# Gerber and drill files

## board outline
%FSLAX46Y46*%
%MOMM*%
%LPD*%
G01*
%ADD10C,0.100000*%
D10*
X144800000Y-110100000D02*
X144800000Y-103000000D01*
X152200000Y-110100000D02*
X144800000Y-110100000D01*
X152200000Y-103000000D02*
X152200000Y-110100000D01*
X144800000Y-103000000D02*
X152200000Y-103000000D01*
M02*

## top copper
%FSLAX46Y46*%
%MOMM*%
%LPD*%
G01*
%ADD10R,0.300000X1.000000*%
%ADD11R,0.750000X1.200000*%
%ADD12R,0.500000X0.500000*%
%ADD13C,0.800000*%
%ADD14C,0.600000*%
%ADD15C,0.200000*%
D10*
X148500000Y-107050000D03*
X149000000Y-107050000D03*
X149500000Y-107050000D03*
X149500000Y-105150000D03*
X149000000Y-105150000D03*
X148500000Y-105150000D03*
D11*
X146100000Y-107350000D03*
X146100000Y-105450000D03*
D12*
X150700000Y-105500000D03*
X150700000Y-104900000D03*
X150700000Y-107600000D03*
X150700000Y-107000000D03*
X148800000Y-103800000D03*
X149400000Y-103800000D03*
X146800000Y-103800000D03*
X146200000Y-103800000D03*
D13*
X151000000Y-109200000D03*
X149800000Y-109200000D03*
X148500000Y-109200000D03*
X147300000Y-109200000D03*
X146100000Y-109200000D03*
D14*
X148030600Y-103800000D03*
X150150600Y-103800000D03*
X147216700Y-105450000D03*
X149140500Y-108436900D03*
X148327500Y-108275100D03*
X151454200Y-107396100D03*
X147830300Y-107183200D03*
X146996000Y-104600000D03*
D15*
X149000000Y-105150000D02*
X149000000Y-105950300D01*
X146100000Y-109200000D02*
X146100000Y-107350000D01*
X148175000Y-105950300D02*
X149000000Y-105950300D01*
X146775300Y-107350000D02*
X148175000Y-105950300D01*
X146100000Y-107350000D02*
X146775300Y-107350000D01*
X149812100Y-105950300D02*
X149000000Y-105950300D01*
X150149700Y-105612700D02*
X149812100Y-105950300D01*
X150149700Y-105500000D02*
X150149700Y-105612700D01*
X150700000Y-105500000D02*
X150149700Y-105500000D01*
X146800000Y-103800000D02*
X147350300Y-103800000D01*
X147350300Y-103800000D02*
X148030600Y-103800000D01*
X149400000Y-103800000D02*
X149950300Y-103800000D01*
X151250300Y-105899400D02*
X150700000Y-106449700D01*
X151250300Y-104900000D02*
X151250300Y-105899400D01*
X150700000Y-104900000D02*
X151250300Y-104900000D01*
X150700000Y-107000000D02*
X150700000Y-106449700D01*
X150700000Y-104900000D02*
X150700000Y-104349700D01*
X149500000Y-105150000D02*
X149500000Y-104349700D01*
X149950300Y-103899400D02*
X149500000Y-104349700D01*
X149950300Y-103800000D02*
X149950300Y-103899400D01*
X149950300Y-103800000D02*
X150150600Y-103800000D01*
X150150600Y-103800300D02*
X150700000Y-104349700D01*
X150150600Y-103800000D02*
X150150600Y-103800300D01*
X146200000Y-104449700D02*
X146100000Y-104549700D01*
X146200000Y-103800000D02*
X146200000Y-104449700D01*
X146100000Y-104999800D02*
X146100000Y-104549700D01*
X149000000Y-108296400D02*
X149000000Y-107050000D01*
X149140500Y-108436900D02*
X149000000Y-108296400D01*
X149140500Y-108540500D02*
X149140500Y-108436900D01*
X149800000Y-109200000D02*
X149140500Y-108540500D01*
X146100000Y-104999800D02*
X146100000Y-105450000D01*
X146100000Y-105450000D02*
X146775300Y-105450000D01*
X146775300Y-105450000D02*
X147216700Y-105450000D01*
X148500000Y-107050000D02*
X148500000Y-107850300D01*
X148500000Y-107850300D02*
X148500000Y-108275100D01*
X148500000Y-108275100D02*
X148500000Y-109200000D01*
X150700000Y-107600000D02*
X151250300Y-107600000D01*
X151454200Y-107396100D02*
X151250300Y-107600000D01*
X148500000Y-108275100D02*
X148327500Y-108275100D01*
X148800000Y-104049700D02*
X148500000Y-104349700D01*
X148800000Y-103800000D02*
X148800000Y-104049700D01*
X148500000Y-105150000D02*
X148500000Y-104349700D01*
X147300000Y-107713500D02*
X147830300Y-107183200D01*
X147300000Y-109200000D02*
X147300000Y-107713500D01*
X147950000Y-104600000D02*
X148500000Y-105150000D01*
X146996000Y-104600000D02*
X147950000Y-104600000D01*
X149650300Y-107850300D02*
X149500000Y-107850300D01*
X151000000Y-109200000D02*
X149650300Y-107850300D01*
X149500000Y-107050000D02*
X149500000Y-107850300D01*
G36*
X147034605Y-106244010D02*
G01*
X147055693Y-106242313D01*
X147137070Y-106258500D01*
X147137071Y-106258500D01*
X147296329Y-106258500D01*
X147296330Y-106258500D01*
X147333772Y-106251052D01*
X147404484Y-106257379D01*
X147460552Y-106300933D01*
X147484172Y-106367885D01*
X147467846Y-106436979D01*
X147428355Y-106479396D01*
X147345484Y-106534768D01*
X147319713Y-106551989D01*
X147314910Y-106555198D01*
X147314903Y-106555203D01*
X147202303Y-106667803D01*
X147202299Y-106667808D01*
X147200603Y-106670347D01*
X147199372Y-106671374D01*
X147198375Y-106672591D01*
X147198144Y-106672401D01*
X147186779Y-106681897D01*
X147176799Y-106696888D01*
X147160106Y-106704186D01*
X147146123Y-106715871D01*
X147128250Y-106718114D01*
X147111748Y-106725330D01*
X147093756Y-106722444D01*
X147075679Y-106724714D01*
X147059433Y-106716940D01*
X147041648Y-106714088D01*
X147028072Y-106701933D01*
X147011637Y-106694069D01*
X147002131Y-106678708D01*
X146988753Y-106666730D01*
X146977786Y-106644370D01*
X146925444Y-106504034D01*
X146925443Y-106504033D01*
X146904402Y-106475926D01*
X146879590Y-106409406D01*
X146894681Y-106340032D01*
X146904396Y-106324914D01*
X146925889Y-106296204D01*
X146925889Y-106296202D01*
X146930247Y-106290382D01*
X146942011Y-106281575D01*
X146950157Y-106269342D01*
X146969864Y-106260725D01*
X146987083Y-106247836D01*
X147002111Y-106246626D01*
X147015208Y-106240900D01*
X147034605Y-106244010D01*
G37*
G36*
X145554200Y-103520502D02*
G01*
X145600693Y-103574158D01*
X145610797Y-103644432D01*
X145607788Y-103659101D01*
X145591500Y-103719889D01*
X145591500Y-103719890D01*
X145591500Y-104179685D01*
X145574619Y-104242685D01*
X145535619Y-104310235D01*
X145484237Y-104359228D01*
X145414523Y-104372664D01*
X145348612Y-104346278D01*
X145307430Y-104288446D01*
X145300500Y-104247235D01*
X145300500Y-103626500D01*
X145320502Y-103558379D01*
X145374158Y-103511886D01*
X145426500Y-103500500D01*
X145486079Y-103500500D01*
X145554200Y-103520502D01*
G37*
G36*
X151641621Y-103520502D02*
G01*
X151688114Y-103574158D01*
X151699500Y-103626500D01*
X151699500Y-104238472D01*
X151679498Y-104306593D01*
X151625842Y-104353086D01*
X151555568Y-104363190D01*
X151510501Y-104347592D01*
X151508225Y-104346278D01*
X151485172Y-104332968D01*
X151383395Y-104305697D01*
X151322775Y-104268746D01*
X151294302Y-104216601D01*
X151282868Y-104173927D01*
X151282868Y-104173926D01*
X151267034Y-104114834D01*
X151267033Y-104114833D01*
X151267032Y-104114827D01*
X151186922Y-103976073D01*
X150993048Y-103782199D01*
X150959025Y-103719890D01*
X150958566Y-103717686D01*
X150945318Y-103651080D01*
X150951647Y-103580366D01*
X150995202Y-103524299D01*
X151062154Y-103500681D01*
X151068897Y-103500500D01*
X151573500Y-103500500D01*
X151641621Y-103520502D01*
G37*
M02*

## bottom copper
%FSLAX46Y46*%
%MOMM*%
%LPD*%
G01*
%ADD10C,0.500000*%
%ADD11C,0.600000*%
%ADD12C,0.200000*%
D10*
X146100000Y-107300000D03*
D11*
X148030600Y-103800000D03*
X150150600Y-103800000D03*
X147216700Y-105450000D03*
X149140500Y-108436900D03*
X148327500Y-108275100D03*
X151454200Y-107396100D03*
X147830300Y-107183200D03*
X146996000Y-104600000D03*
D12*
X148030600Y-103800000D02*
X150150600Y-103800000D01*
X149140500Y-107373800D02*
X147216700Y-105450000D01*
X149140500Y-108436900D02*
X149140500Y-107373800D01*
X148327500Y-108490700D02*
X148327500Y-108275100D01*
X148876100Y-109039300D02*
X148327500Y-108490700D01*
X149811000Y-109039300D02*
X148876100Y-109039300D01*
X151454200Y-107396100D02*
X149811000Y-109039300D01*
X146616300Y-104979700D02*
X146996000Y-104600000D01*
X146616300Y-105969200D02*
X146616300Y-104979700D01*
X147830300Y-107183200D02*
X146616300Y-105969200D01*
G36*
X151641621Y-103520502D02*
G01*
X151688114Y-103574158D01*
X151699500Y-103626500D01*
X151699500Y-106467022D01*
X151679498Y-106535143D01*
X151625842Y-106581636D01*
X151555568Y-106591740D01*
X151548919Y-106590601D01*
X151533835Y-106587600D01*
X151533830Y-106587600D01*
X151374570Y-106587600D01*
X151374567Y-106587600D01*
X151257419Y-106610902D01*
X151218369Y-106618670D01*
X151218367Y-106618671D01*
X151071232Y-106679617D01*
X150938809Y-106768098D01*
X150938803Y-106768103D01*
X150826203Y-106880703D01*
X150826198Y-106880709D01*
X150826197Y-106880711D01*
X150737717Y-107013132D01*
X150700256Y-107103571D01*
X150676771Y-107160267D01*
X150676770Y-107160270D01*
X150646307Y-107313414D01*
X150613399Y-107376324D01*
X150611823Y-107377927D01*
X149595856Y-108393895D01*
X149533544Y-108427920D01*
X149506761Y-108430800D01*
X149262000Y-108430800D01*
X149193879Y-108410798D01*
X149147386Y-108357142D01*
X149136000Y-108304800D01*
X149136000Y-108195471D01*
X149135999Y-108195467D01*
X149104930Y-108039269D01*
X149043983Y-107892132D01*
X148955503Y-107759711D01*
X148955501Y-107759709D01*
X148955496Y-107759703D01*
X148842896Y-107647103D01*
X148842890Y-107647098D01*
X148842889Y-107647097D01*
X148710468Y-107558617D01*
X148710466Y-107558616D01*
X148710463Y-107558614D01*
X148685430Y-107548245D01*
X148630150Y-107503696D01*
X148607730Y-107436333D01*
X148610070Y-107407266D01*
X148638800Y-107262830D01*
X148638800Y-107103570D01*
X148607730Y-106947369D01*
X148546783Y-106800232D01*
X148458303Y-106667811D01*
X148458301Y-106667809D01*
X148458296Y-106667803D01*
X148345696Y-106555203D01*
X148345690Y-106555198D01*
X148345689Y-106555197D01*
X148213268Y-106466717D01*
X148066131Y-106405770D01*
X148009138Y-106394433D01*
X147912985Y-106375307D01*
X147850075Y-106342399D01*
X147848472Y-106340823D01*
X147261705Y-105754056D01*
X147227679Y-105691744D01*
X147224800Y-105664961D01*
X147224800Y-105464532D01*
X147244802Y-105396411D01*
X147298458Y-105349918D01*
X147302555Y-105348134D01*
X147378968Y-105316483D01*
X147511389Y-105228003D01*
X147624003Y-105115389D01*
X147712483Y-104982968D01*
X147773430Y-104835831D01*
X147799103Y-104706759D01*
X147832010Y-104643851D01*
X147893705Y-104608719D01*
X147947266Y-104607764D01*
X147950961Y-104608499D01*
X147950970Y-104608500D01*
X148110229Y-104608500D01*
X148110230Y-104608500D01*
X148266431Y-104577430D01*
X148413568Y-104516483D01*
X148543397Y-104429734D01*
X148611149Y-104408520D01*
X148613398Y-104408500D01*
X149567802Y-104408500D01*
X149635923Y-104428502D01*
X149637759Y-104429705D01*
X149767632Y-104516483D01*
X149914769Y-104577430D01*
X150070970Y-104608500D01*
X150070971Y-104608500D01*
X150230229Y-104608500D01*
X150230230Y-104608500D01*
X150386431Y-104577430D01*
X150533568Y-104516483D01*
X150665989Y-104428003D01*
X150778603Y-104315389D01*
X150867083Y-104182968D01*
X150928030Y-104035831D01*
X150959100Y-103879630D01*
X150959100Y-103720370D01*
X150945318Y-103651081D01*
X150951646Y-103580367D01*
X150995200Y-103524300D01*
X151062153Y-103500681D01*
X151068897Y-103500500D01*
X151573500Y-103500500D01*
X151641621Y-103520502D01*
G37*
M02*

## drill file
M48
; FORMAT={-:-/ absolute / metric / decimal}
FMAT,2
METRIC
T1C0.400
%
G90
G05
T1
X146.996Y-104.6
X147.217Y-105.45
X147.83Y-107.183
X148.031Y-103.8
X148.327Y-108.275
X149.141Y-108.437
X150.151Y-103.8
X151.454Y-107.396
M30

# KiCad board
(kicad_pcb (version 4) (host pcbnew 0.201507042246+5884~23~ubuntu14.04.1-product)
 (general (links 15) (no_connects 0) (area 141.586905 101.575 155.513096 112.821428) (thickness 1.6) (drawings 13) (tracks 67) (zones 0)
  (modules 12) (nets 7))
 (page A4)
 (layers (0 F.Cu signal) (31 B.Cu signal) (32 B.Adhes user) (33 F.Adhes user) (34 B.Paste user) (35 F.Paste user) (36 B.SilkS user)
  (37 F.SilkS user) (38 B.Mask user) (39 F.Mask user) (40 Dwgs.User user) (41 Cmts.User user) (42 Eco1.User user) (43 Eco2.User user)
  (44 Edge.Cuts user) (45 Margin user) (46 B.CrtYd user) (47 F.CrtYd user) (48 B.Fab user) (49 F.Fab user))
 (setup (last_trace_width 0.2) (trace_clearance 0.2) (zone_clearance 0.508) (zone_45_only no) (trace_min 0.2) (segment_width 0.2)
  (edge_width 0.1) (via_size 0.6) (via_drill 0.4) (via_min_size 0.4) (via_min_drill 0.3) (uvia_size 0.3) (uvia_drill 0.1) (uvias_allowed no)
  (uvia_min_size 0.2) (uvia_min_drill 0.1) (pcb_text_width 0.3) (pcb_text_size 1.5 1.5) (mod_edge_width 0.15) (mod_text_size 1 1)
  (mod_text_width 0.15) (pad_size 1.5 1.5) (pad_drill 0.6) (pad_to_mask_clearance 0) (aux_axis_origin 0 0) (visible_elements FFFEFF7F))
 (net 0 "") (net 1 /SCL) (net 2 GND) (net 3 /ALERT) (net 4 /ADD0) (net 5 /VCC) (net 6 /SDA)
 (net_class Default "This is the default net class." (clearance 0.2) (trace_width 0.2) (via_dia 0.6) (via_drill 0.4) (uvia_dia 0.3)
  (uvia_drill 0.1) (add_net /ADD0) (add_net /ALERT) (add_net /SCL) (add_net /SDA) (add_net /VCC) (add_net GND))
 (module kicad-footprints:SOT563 (layer F.Cu) (at 149 106.1)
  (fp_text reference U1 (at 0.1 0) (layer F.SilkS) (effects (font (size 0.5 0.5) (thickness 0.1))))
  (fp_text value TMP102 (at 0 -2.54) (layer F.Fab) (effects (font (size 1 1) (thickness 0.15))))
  (pad 1 smd rect (at -0.5 0.95) (size 0.3 1) (layers F.Cu F.Paste F.Mask) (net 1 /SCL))
  (pad 2 smd rect (at 0 0.95) (size 0.3 1) (layers F.Cu F.Paste F.Mask) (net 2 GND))
  (pad 3 smd rect (at 0.5 0.95) (size 0.3 1) (layers F.Cu F.Paste F.Mask) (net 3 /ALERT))
  (pad 4 smd rect (at 0.5 -0.95) (size 0.3 1) (layers F.Cu F.Paste F.Mask) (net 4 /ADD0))
  (pad 5 smd rect (at 0 -0.95) (size 0.3 1) (layers F.Cu F.Paste F.Mask) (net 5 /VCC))
  (pad 6 smd rect (at -0.5 -0.95) (size 0.3 1) (layers F.Cu F.Paste F.Mask) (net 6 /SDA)))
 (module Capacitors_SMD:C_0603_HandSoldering (layer F.Cu) (at 146.1 106.4 90)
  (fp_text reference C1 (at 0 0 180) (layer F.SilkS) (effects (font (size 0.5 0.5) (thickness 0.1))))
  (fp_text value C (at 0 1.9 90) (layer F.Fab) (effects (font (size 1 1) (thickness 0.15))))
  (pad 1 smd rect (at -0.95 0 90) (size 1.2 0.75) (layers F.Cu F.Paste F.Mask) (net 5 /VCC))
  (pad 2 smd rect (at 0.95 0 90) (size 1.2 0.75) (layers F.Cu F.Paste F.Mask) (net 2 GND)))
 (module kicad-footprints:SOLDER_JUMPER (layer F.Cu) (at 150.7 105.2 90)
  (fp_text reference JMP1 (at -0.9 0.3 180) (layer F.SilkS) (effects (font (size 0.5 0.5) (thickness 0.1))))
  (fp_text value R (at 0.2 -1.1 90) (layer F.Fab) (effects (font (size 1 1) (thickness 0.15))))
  (pad 1 smd rect (at -0.3 0 90) (size 0.5 0.5) (layers F.Cu F.Paste F.Mask) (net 5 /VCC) (clearance 0.05))
  (pad 2 smd rect (at 0.3 0 90) (size 0.5 0.5) (layers F.Cu F.Paste F.Mask) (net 4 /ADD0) (clearance 0.05)))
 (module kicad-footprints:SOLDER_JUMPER (layer F.Cu) (at 150.7 107.3 90)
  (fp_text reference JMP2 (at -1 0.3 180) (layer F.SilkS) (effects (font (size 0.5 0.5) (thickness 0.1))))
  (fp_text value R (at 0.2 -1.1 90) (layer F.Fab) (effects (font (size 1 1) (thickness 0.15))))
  (pad 1 smd rect (at -0.3 0 90) (size 0.5 0.5) (layers F.Cu F.Paste F.Mask) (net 1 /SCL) (clearance 0.05))
  (pad 2 smd rect (at 0.3 0 90) (size 0.5 0.5) (layers F.Cu F.Paste F.Mask) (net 4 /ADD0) (clearance 0.05)))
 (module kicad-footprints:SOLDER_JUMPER (layer F.Cu) (at 149.1 103.8)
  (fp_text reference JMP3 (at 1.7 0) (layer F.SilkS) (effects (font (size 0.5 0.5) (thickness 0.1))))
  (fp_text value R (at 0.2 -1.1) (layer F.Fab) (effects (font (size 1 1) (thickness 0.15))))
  (pad 1 smd rect (at -0.3 0) (size 0.5 0.5) (layers F.Cu F.Paste F.Mask) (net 6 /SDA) (clearance 0.05))
  (pad 2 smd rect (at 0.3 0) (size 0.5 0.5) (layers F.Cu F.Paste F.Mask) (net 4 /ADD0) (clearance 0.05)))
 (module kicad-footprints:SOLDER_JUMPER (layer F.Cu) (at 146.5 103.8 180)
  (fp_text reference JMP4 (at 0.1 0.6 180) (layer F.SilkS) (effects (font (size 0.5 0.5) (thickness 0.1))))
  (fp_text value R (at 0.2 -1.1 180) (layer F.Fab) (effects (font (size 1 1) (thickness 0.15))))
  (pad 1 smd rect (at -0.3 0 180) (size 0.5 0.5) (layers F.Cu F.Paste F.Mask) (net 4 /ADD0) (clearance 0.05))
  (pad 2 smd rect (at 0.3 0 180) (size 0.5 0.5) (layers F.Cu F.Paste F.Mask) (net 2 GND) (clearance 0.05)))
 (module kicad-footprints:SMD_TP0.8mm (layer F.Cu) (at 151 109.2)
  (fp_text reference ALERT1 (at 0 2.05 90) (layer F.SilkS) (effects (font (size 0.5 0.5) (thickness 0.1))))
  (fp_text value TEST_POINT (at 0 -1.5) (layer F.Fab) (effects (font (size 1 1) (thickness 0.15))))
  (pad 1 smd circle (at 0 0) (size 0.8 0.8) (layers F.Cu F.Paste F.Mask) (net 3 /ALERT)))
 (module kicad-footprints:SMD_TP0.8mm (layer F.Cu) (at 149.8 109.2)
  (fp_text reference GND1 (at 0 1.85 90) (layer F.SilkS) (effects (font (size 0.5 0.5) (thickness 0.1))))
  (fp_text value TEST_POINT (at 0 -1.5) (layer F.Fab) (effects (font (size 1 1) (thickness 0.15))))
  (pad 1 smd circle (at 0 0) (size 0.8 0.8) (layers F.Cu F.Paste F.Mask) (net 2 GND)))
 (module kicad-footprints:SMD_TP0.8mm (layer F.Cu) (at 148.5 109.2)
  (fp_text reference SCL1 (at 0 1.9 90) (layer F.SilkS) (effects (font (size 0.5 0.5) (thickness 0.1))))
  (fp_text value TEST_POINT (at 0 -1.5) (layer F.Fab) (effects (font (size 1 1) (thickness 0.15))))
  (pad 1 smd circle (at 0 0) (size 0.8 0.8) (layers F.Cu F.Paste F.Mask) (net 1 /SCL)))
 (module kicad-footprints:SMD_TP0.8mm (layer F.Cu) (at 147.3 109.2)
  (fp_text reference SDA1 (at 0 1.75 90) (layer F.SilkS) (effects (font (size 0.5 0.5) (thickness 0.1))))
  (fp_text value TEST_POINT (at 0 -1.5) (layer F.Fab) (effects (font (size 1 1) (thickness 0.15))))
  (pad 1 smd circle (at 0 0) (size 0.8 0.8) (layers F.Cu F.Paste F.Mask) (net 6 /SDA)))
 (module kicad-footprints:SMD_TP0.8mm (layer F.Cu) (at 146.1 109.2)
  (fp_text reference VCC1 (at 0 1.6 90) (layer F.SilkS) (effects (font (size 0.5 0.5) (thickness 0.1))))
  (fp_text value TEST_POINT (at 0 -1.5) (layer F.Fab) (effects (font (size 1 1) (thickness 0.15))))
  (pad 1 smd circle (at 0 0) (size 0.8 0.8) (layers F.Cu F.Paste F.Mask) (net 5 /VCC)))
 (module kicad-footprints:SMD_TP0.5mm (layer B.Cu) (at 146.1 107.3)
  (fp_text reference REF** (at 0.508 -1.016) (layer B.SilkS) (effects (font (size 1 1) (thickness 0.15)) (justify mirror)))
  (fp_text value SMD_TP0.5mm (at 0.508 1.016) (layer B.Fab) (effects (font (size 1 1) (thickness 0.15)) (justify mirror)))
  (pad 1 smd circle (at 0 0) (size 0.5 0.5) (layers B.Cu B.Paste B.Mask)))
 (gr_line (start 144.8 110.1) (end 144.8 103) (angle 90) (layer Edge.Cuts) (width 0.1))
 (gr_line (start 152.2 110.1) (end 144.8 110.1) (angle 90) (layer Edge.Cuts) (width 0.1))
 (gr_line (start 152.2 103) (end 152.2 110.1) (angle 90) (layer Edge.Cuts) (width 0.1))
 (gr_line (start 144.8 103) (end 152.2 103) (angle 90) (layer Edge.Cuts) (width 0.1))
 (segment (start 149 105.15) (end 149 105.9503) (width 0.2) (layer F.Cu) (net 5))
 (segment (start 146.1 109.2) (end 146.1 107.35) (width 0.2) (layer F.Cu) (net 5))
 (segment (start 148.175 105.9503) (end 149 105.9503) (width 0.2) (layer F.Cu) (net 5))
 (segment (start 146.7753 107.35) (end 148.175 105.9503) (width 0.2) (layer F.Cu) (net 5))
 (segment (start 146.1 107.35) (end 146.7753 107.35) (width 0.2) (layer F.Cu) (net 5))
 (segment (start 149.8121 105.9503) (end 149 105.9503) (width 0.2) (layer F.Cu) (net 5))
 (segment (start 150.1497 105.6127) (end 149.8121 105.9503) (width 0.2) (layer F.Cu) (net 5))
 (segment (start 150.1497 105.5) (end 150.1497 105.6127) (width 0.2) (layer F.Cu) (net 5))
 (segment (start 150.7 105.5) (end 150.1497 105.5) (width 0.2) (layer F.Cu) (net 5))
 (via (at 148.0306 103.8) (size 0.6) (layers F.Cu B.Cu) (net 4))
 (via (at 150.1506 103.8) (size 0.6) (layers F.Cu B.Cu) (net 4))
 (segment (start 146.8 103.8) (end 147.3503 103.8) (width 0.2) (layer F.Cu) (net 4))
 (segment (start 148.0306 103.8) (end 150.1506 103.8) (width 0.2) (layer B.Cu) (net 4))
 (segment (start 147.3503 103.8) (end 148.0306 103.8) (width 0.2) (layer F.Cu) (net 4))
 (segment (start 149.4 103.8) (end 149.9503 103.8) (width 0.2) (layer F.Cu) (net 4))
 (segment (start 151.2503 105.8994) (end 150.7 106.4497) (width 0.2) (layer F.Cu) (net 4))
 (segment (start 151.2503 104.9) (end 151.2503 105.8994) (width 0.2) (layer F.Cu) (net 4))
 (segment (start 150.7 104.9) (end 151.2503 104.9) (width 0.2) (layer F.Cu) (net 4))
 (segment (start 150.7 107) (end 150.7 106.4497) (width 0.2) (layer F.Cu) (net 4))
 (segment (start 150.7 104.9) (end 150.7 104.3497) (width 0.2) (layer F.Cu) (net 4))
 (segment (start 149.5 105.15) (end 149.5 104.3497) (width 0.2) (layer F.Cu) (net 4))
 (segment (start 149.9503 103.8994) (end 149.5 104.3497) (width 0.2) (layer F.Cu) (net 4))
 (segment (start 149.9503 103.8) (end 149.9503 103.8994) (width 0.2) (layer F.Cu) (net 4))
 (segment (start 149.9503 103.8) (end 150.1506 103.8) (width 0.2) (layer F.Cu) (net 4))
 (segment (start 150.1506 103.8003) (end 150.7 104.3497) (width 0.2) (layer F.Cu) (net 4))
 (segment (start 150.1506 103.8) (end 150.1506 103.8003) (width 0.2) (layer F.Cu) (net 4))
 (via (at 147.2167 105.45) (size 0.6) (layers F.Cu B.Cu) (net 2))
 (via (at 149.1405 108.4369) (size 0.6) (layers F.Cu B.Cu) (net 2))
 (segment (start 146.2 104.4497) (end 146.1 104.5497) (width 0.2) (layer F.Cu) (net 2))
 (segment (start 146.2 103.8) (end 146.2 104.4497) (width 0.2) (layer F.Cu) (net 2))
 (segment (start 146.1 104.9998) (end 146.1 104.5497) (width 0.2) (layer F.Cu) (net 2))
 (segment (start 149 108.2964) (end 149 107.05) (width 0.2) (layer F.Cu) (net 2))
 (segment (start 149.1405 108.4369) (end 149 108.2964) (width 0.2) (layer F.Cu) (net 2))
 (segment (start 149.1405 108.5405) (end 149.1405 108.4369) (width 0.2) (layer F.Cu) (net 2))
 (segment (start 149.8 109.2) (end 149.1405 108.5405) (width 0.2) (layer F.Cu) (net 2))
 (segment (start 146.1 104.9998) (end 146.1 105.45) (width 0.2) (layer F.Cu) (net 2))
 (segment (start 146.1 105.45) (end 146.7753 105.45) (width 0.2) (layer F.Cu) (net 2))
 (segment (start 149.1405 107.3738) (end 147.2167 105.45) (width 0.2) (layer B.Cu) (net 2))
 (segment (start 149.1405 108.4369) (end 149.1405 107.3738) (width 0.2) (layer B.Cu) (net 2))
 (segment (start 146.7753 105.45) (end 147.2167 105.45) (width 0.2) (layer F.Cu) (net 2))
 (via (at 148.3275 108.2751) (size 0.6) (layers F.Cu B.Cu) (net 1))
 (via (at 151.4542 107.3961) (size 0.6) (layers F.Cu B.Cu) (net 1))
 (segment (start 148.5 107.05) (end 148.5 107.8503) (width 0.2) (layer F.Cu) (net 1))
 (segment (start 148.5 107.8503) (end 148.5 108.2751) (width 0.2) (layer F.Cu) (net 1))
 (segment (start 148.5 108.2751) (end 148.5 109.2) (width 0.2) (layer F.Cu) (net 1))
 (segment (start 150.7 107.6) (end 151.2503 107.6) (width 0.2) (layer F.Cu) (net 1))
 (segment (start 151.4542 107.3961) (end 151.2503 107.6) (width 0.2) (layer F.Cu) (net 1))
 (segment (start 148.3275 108.4907) (end 148.3275 108.2751) (width 0.2) (layer B.Cu) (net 1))
 (segment (start 148.8761 109.0393) (end 148.3275 108.4907) (width 0.2) (layer B.Cu) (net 1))
 (segment (start 149.811 109.0393) (end 148.8761 109.0393) (width 0.2) (layer B.Cu) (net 1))
 (segment (start 151.4542 107.3961) (end 149.811 109.0393) (width 0.2) (layer B.Cu) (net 1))
 (segment (start 148.5 108.2751) (end 148.3275 108.2751) (width 0.2) (layer F.Cu) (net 1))
 (via (at 147.8303 107.1832) (size 0.6) (layers F.Cu B.Cu) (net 6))
 (via (at 146.996 104.6) (size 0.6) (layers F.Cu B.Cu) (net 6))
 (segment (start 148.8 104.0497) (end 148.5 104.3497) (width 0.2) (layer F.Cu) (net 6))
 (segment (start 148.8 103.8) (end 148.8 104.0497) (width 0.2) (layer F.Cu) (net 6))
 (segment (start 148.5 105.15) (end 148.5 104.3497) (width 0.2) (layer F.Cu) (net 6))
 (segment (start 147.3 107.7135) (end 147.8303 107.1832) (width 0.2) (layer F.Cu) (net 6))
 (segment (start 147.3 109.2) (end 147.3 107.7135) (width 0.2) (layer F.Cu) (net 6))
 (segment (start 146.6163 104.9797) (end 146.996 104.6) (width 0.2) (layer B.Cu) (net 6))
 (segment (start 146.6163 105.9692) (end 146.6163 104.9797) (width 0.2) (layer B.Cu) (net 6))
 (segment (start 147.8303 107.1832) (end 146.6163 105.9692) (width 0.2) (layer B.Cu) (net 6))
 (segment (start 147.95 104.6) (end 148.5 105.15) (width 0.2) (layer F.Cu) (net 6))
 (segment (start 146.996 104.6) (end 147.95 104.6) (width 0.2) (layer F.Cu) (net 6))
 (segment (start 149.6503 107.8503) (end 149.5 107.8503) (width 0.2) (layer F.Cu) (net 3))
 (segment (start 151 109.2) (end 149.6503 107.8503) (width 0.2) (layer F.Cu) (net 3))
 (segment (start 149.5 107.05) (end 149.5 107.8503) (width 0.2) (layer F.Cu) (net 3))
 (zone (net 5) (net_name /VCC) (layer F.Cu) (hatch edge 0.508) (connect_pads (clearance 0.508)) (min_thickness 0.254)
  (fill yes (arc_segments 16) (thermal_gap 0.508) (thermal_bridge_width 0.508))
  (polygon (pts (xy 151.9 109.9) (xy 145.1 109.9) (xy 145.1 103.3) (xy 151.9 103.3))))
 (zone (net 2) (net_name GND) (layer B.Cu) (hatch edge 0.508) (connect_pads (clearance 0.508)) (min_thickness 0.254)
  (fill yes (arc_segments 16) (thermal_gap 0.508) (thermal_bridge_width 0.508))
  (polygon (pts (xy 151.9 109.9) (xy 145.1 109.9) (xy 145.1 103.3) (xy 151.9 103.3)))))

